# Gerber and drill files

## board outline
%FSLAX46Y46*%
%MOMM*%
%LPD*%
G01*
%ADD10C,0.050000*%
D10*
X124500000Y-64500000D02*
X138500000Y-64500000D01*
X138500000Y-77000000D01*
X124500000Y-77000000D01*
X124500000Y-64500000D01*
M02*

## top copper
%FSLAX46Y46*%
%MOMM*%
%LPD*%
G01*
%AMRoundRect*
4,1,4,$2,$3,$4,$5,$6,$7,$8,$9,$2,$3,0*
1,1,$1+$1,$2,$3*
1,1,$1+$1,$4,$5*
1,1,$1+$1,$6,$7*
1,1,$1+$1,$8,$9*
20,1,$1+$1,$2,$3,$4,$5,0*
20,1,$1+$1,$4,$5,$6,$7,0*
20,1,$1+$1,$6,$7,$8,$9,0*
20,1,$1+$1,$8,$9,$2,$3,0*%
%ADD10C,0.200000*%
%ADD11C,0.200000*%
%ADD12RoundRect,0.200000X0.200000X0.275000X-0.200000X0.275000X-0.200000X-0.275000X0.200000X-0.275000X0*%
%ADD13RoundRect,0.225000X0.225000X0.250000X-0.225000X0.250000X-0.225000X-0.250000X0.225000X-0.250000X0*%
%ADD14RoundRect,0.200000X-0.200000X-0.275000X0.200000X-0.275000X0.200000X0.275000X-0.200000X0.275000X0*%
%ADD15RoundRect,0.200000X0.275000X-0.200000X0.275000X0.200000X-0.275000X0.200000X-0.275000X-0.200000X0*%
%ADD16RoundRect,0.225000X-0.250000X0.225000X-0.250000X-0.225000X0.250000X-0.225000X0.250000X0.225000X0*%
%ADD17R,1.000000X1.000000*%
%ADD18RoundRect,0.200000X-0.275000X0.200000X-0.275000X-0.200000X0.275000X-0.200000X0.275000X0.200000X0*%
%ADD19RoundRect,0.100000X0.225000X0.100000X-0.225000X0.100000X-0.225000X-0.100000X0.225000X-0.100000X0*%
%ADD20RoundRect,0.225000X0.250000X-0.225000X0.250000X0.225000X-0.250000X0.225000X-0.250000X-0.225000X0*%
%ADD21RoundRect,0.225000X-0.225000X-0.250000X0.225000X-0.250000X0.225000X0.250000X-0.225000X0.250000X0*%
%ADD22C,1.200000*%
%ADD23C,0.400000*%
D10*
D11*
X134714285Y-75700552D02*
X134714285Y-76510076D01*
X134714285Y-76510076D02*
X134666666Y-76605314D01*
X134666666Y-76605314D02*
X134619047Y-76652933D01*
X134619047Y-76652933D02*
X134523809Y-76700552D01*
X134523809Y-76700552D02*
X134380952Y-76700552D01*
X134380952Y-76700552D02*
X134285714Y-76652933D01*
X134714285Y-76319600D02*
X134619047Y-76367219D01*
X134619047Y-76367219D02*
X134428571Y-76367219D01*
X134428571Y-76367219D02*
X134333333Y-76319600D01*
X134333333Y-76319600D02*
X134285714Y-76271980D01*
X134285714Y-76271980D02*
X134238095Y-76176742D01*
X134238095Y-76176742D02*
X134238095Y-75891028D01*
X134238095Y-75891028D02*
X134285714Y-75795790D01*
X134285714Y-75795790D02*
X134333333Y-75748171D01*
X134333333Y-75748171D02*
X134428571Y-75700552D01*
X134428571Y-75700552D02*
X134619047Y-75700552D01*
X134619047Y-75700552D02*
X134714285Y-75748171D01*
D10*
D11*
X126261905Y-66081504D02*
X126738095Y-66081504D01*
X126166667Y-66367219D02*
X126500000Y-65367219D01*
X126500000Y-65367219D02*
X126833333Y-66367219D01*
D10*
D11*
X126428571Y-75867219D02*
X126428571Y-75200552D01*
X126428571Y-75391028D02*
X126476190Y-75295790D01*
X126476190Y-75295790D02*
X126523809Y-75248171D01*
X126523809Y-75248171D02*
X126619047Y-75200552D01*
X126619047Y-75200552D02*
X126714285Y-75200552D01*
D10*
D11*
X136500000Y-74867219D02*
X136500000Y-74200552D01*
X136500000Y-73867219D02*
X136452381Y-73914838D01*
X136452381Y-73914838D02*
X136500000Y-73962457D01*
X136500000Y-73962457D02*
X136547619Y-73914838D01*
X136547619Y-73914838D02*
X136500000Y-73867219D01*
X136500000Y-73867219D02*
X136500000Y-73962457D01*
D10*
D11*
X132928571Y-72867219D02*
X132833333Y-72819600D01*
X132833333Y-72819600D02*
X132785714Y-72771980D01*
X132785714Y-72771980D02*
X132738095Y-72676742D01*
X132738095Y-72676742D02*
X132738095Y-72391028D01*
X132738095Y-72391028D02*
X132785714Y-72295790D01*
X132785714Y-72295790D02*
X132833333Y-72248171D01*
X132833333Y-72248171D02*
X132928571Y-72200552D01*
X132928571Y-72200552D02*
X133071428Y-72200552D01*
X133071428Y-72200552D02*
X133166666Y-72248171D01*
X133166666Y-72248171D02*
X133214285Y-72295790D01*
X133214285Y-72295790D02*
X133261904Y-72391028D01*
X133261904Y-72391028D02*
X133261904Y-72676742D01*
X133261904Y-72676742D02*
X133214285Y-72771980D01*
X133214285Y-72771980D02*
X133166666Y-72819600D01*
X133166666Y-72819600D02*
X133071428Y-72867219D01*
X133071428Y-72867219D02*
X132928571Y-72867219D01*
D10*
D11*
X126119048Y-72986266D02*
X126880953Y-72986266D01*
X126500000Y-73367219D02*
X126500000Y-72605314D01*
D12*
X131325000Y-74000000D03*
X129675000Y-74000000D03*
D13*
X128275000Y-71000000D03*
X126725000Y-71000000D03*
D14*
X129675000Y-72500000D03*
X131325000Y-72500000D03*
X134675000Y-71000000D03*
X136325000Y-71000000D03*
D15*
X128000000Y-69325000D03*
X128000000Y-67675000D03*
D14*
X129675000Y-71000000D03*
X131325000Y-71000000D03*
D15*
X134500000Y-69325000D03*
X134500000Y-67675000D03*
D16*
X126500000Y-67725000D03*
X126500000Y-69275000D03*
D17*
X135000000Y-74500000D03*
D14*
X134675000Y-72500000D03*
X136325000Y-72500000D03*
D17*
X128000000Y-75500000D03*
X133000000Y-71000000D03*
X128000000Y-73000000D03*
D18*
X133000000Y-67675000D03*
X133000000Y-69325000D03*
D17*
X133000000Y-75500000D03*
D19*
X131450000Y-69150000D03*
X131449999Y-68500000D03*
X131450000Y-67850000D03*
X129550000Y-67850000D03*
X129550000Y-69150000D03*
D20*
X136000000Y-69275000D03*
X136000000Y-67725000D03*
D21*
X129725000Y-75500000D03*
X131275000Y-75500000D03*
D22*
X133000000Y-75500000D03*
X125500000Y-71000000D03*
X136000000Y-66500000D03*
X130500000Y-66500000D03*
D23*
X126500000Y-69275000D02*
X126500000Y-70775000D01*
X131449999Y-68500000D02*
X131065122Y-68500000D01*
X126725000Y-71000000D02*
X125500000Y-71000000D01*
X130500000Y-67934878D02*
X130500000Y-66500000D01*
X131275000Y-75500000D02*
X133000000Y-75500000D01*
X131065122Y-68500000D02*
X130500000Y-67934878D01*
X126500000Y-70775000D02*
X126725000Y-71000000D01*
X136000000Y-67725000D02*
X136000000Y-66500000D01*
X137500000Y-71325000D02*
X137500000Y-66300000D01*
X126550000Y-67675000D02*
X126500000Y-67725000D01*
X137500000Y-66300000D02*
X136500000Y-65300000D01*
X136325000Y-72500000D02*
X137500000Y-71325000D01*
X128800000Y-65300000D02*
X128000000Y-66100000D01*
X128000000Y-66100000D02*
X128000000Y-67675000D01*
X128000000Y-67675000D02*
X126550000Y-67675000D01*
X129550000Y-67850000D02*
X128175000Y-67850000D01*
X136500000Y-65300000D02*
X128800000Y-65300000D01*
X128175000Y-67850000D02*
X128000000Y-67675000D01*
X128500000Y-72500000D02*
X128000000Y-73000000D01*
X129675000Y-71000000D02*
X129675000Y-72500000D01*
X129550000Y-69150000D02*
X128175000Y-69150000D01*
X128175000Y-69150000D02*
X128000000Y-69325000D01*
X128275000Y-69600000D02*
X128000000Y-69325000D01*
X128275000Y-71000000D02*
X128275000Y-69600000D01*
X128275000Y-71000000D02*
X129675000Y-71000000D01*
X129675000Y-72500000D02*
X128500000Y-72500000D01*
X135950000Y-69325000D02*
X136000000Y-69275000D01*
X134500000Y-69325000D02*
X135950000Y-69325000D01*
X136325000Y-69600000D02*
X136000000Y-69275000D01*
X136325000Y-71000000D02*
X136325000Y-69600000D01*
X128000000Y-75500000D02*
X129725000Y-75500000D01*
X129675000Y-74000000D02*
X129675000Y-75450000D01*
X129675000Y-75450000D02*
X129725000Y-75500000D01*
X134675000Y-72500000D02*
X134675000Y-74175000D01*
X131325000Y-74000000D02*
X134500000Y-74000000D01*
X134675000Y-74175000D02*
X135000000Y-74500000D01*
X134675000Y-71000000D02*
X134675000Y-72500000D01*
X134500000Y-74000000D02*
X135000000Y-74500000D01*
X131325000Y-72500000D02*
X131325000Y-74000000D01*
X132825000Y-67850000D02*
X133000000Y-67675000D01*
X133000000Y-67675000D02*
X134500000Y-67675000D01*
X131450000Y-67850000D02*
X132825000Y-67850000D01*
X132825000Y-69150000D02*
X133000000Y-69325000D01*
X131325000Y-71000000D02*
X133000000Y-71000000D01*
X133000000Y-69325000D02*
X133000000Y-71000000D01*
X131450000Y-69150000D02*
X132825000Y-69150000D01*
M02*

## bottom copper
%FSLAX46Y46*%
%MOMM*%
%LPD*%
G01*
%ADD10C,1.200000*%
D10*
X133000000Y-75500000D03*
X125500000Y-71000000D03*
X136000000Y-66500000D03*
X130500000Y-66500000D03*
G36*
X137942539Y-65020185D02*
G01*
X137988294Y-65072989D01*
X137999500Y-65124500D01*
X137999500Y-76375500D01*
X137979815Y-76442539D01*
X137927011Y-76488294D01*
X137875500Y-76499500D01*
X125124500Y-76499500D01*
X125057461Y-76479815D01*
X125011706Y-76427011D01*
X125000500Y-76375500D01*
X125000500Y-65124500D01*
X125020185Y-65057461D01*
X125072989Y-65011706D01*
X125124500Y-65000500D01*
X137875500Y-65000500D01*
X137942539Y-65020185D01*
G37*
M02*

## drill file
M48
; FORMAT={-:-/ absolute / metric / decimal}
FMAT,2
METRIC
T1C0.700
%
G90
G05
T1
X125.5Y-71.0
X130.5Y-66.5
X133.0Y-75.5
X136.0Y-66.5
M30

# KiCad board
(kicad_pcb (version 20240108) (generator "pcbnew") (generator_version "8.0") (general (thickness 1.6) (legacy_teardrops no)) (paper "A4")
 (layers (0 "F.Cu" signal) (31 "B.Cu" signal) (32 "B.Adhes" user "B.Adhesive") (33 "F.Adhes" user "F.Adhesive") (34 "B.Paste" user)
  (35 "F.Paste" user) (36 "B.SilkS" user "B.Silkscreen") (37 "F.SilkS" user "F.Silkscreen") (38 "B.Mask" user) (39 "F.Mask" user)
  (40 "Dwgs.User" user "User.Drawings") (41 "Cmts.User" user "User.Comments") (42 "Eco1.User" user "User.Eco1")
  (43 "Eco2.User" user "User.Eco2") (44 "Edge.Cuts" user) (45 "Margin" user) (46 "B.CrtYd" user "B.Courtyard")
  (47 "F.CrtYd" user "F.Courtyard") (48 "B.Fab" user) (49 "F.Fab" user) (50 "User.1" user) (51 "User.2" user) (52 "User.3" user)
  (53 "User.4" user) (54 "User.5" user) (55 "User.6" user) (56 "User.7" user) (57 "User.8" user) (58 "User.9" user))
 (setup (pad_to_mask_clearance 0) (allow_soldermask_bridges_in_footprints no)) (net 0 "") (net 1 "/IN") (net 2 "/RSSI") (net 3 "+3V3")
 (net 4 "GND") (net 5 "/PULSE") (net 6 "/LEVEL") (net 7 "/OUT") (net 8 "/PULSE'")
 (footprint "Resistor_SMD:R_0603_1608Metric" (layer "F.Cu") (at 130.5 74 180)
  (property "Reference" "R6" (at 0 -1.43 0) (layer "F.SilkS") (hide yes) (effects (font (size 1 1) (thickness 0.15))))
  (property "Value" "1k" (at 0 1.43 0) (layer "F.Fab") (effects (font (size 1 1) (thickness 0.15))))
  (pad "1" smd roundrect (at -0.825 0 180) (size 0.8 0.95) (layers "F.Cu" "F.Paste" "F.Mask") (roundrect_rratio 0.25) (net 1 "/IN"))
  (pad "2" smd roundrect (at 0.825 0 180) (size 0.8 0.95) (layers "F.Cu" "F.Paste" "F.Mask") (roundrect_rratio 0.25) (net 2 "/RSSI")))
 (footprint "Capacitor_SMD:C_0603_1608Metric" (layer "F.Cu") (at 127.5 71 180)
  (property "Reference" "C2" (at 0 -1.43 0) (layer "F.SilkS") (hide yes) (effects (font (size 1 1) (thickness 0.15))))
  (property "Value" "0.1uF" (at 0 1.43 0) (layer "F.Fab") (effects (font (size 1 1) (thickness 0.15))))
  (pad "1" smd roundrect (at -0.775 0 180) (size 0.9 0.95) (layers "F.Cu" "F.Paste" "F.Mask") (roundrect_rratio 0.25) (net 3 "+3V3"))
  (pad "2" smd roundrect (at 0.775 0 180) (size 0.9 0.95) (layers "F.Cu" "F.Paste" "F.Mask") (roundrect_rratio 0.25) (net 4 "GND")))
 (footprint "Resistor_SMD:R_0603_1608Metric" (layer "F.Cu") (at 130.5 72.5)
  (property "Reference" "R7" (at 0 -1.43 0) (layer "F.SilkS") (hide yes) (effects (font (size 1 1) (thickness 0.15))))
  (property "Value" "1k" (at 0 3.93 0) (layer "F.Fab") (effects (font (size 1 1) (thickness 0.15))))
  (pad "1" smd roundrect (at -0.825 0) (size 0.8 0.95) (layers "F.Cu" "F.Paste" "F.Mask") (roundrect_rratio 0.25) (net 3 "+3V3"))
  (pad "2" smd roundrect (at 0.825 0) (size 0.8 0.95) (layers "F.Cu" "F.Paste" "F.Mask") (roundrect_rratio 0.25) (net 1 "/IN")))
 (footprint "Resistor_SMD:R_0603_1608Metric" (layer "F.Cu") (at 135.5 71)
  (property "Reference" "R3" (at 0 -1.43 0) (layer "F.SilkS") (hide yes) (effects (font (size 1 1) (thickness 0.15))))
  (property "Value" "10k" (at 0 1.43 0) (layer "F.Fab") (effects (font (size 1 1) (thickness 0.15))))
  (pad "1" smd roundrect (at -0.825 0) (size 0.8 0.95) (layers "F.Cu" "F.Paste" "F.Mask") (roundrect_rratio 0.25) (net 1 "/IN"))
  (pad "2" smd roundrect (at 0.825 0) (size 0.8 0.95) (layers "F.Cu" "F.Paste" "F.Mask") (roundrect_rratio 0.25) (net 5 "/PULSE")))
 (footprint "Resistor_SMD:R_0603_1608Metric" (layer "F.Cu") (at 128 68.5 90)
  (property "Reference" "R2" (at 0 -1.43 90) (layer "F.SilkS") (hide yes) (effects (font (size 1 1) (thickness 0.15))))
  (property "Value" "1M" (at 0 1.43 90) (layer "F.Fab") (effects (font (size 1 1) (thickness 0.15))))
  (pad "1" smd roundrect (at -0.825 0 90) (size 0.8 0.95) (layers "F.Cu" "F.Paste" "F.Mask") (roundrect_rratio 0.25) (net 3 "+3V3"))
  (pad "2" smd roundrect (at 0.825 0 90) (size 0.8 0.95) (layers "F.Cu" "F.Paste" "F.Mask") (roundrect_rratio 0.25) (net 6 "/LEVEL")))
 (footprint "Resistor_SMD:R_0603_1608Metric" (layer "F.Cu") (at 130.5 71)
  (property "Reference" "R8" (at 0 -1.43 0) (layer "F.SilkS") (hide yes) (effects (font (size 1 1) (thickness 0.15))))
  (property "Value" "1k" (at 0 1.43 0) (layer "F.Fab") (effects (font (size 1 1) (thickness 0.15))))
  (pad "1" smd roundrect (at -0.825 0) (size 0.8 0.95) (layers "F.Cu" "F.Paste" "F.Mask") (roundrect_rratio 0.25) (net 3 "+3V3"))
  (pad "2" smd roundrect (at 0.825 0) (size 0.8 0.95) (layers "F.Cu" "F.Paste" "F.Mask") (roundrect_rratio 0.25) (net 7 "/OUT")))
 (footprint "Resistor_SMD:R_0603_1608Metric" (layer "F.Cu") (at 134.5 68.5 90)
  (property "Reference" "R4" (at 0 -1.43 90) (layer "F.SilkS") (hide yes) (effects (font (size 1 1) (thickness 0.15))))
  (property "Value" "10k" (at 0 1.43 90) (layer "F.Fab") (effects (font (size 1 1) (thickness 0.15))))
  (pad "1" smd roundrect (at -0.825 0 90) (size 0.8 0.95) (layers "F.Cu" "F.Paste" "F.Mask") (roundrect_rratio 0.25) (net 5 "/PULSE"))
  (pad "2" smd roundrect (at 0.825 0 90) (size 0.8 0.95) (layers "F.Cu" "F.Paste" "F.Mask") (roundrect_rratio 0.25) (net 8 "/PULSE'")))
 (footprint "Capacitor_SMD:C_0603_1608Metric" (layer "F.Cu") (at 126.5 68.5 -90)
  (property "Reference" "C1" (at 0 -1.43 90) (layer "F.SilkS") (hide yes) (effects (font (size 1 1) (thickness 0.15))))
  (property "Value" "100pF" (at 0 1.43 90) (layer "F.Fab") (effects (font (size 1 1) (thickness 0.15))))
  (pad "1" smd roundrect (at -0.775 0 270) (size 0.9 0.95) (layers "F.Cu" "F.Paste" "F.Mask") (roundrect_rratio 0.25) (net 6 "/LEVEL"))
  (pad "2" smd roundrect (at 0.775 0 270) (size 0.9 0.95) (layers "F.Cu" "F.Paste" "F.Mask") (roundrect_rratio 0.25) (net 4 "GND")))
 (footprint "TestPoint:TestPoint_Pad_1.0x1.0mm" (layer "F.Cu") (at 135 74.5)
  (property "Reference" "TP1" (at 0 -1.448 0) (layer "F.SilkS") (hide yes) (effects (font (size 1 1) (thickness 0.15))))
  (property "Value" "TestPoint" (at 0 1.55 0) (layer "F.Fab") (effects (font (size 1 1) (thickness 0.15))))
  (pad "1" smd rect (at 0 0) (size 1 1) (layers "F.Cu" "F.Mask") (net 1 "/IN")))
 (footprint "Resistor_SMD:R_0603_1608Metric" (layer "F.Cu") (at 135.5 72.5)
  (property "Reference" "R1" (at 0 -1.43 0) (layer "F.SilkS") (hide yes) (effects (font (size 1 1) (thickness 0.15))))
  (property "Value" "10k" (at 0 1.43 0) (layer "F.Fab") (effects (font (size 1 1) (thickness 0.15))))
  (pad "1" smd roundrect (at -0.825 0) (size 0.8 0.95) (layers "F.Cu" "F.Paste" "F.Mask") (roundrect_rratio 0.25) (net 1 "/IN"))
  (pad "2" smd roundrect (at 0.825 0) (size 0.8 0.95) (layers "F.Cu" "F.Paste" "F.Mask") (roundrect_rratio 0.25) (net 6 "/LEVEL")))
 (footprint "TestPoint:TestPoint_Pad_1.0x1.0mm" (layer "F.Cu") (at 128 75.5)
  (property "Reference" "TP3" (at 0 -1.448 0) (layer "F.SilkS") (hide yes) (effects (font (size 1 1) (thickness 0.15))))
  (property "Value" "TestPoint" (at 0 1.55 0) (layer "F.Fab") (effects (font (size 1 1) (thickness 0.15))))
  (pad "1" smd rect (at 0 0) (size 1 1) (layers "F.Cu" "F.Mask") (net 2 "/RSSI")))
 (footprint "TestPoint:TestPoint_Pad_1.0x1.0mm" (layer "F.Cu") (at 133 71)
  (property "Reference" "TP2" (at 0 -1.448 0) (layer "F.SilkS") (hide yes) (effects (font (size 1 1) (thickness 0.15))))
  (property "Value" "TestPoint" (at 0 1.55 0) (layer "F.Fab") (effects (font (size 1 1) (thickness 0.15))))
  (pad "1" smd rect (at 0 0) (size 1 1) (layers "F.Cu" "F.Mask") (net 7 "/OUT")))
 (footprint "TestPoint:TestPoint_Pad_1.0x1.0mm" (layer "F.Cu") (at 128 73)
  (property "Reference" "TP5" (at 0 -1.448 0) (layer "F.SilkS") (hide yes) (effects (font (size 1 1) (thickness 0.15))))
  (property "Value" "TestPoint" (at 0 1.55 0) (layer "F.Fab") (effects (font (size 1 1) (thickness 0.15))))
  (pad "1" smd rect (at 0 0) (size 1 1) (layers "F.Cu" "F.Mask") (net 3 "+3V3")))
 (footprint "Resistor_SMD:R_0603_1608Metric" (layer "F.Cu") (at 133 68.5 -90)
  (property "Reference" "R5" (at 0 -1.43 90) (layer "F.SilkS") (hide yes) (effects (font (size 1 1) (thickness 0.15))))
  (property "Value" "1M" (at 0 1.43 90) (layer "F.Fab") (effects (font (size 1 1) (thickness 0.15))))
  (pad "1" smd roundrect (at -0.825 0 270) (size 0.8 0.95) (layers "F.Cu" "F.Paste" "F.Mask") (roundrect_rratio 0.25) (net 8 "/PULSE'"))
  (pad "2" smd roundrect (at 0.825 0 270) (size 0.8 0.95) (layers "F.Cu" "F.Paste" "F.Mask") (roundrect_rratio 0.25) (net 7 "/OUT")))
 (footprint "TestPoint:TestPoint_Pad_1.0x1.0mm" (layer "F.Cu") (at 133 75.5)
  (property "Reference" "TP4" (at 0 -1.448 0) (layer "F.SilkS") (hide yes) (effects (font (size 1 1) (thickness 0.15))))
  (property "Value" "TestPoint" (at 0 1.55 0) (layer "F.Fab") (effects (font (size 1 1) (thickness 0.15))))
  (pad "1" smd rect (at 0 0) (size 1 1) (layers "F.Cu" "F.Mask") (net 4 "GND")))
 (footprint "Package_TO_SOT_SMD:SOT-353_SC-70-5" (layer "F.Cu") (at 130.5 68.5 180)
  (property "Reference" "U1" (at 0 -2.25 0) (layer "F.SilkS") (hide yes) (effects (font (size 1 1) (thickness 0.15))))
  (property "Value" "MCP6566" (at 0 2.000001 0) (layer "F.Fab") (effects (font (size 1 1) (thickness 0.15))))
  (pad "1" smd roundrect (at -0.95 -0.65 180) (size 0.65 0.4) (layers "F.Cu" "F.Paste" "F.Mask") (roundrect_rratio 0.25) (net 7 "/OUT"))
  (pad "2" smd roundrect (at -0.949999 0 180) (size 0.65 0.4) (layers "F.Cu" "F.Paste" "F.Mask") (roundrect_rratio 0.25) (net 4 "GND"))
  (pad "3" smd roundrect (at -0.95 0.65 180) (size 0.65 0.4) (layers "F.Cu" "F.Paste" "F.Mask") (roundrect_rratio 0.25) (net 8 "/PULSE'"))
  (pad "4" smd roundrect (at 0.95 0.65 180) (size 0.65 0.4) (layers "F.Cu" "F.Paste" "F.Mask") (roundrect_rratio 0.25) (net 6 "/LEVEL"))
  (pad "5" smd roundrect (at 0.95 -0.65 180) (size 0.65 0.4) (layers "F.Cu" "F.Paste" "F.Mask") (roundrect_rratio 0.25) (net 3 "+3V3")))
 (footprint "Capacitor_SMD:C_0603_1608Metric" (layer "F.Cu") (at 136 68.5 90)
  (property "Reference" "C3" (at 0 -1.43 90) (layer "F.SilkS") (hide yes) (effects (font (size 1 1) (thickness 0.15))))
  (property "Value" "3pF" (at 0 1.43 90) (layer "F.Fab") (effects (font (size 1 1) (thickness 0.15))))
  (pad "1" smd roundrect (at -0.775 0 90) (size 0.9 0.95) (layers "F.Cu" "F.Paste" "F.Mask") (roundrect_rratio 0.25) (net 5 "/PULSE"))
  (pad "2" smd roundrect (at 0.775 0 90) (size 0.9 0.95) (layers "F.Cu" "F.Paste" "F.Mask") (roundrect_rratio 0.25) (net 4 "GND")))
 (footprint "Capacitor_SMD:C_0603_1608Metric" (layer "F.Cu") (at 130.5 75.5)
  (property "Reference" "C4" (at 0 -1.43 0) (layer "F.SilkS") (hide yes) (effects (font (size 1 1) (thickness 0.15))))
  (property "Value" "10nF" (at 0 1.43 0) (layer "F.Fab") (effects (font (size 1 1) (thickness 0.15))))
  (pad "1" smd roundrect (at -0.775 0) (size 0.9 0.95) (layers "F.Cu" "F.Paste" "F.Mask") (roundrect_rratio 0.25) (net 2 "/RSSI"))
  (pad "2" smd roundrect (at 0.775 0) (size 0.9 0.95) (layers "F.Cu" "F.Paste" "F.Mask") (roundrect_rratio 0.25) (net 4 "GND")))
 (gr_rect (start 124.5 64.5) (end 138.5 77) (stroke (width 0.05) (type default)) (fill none) (layer "Edge.Cuts"))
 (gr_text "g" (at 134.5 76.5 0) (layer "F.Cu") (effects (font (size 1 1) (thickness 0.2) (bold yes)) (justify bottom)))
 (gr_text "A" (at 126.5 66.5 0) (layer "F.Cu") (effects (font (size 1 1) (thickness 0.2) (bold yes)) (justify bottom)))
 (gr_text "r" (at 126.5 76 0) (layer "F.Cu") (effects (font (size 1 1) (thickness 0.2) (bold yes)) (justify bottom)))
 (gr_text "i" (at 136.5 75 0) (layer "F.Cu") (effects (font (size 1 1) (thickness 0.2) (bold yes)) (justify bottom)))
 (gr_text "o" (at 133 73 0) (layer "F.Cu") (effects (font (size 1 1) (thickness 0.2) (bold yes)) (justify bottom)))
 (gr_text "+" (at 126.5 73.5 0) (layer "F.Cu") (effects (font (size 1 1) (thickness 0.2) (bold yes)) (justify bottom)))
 (segment (start 126.5 69.275) (end 126.5 70.775) (width 0.4) (layer "F.Cu") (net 4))
 (segment (start 131.449999 68.5) (end 131.065122 68.5) (width 0.4) (layer "F.Cu") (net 4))
 (segment (start 126.725 71) (end 125.5 71) (width 0.4) (layer "F.Cu") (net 4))
 (segment (start 130.5 67.934878) (end 130.5 66.5) (width 0.4) (layer "F.Cu") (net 4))
 (segment (start 131.275 75.5) (end 133 75.5) (width 0.4) (layer "F.Cu") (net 4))
 (segment (start 131.065122 68.5) (end 130.5 67.934878) (width 0.4) (layer "F.Cu") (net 4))
 (segment (start 126.5 70.775) (end 126.725 71) (width 0.4) (layer "F.Cu") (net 4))
 (segment (start 136 67.725) (end 136 66.5) (width 0.4) (layer "F.Cu") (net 4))
 (via (at 133 75.5) (size 1.2) (drill 0.7) (layers "F.Cu" "B.Cu") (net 4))
 (via (at 125.5 71) (size 1.2) (drill 0.7) (layers "F.Cu" "B.Cu") (free yes) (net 4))
 (via (at 136 66.5) (size 1.2) (drill 0.7) (layers "F.Cu" "B.Cu") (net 4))
 (via (at 130.5 66.5) (size 1.2) (drill 0.7) (layers "F.Cu" "B.Cu") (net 4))
 (segment (start 137.5 71.325) (end 137.5 66.3) (width 0.4) (layer "F.Cu") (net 6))
 (segment (start 126.55 67.675) (end 126.5 67.725) (width 0.4) (layer "F.Cu") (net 6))
 (segment (start 137.5 66.3) (end 136.5 65.3) (width 0.4) (layer "F.Cu") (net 6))
 (segment (start 136.325 72.5) (end 137.5 71.325) (width 0.4) (layer "F.Cu") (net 6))
 (segment (start 128.8 65.3) (end 128 66.1) (width 0.4) (layer "F.Cu") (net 6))
 (segment (start 128 66.1) (end 128 67.675) (width 0.4) (layer "F.Cu") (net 6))
 (segment (start 128 67.675) (end 126.55 67.675) (width 0.4) (layer "F.Cu") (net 6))
 (segment (start 129.55 67.85) (end 128.175 67.85) (width 0.4) (layer "F.Cu") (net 6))
 (segment (start 136.5 65.3) (end 128.8 65.3) (width 0.4) (layer "F.Cu") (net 6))
 (segment (start 128.175 67.85) (end 128 67.675) (width 0.4) (layer "F.Cu") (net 6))
 (segment (start 128.5 72.5) (end 128 73) (width 0.4) (layer "F.Cu") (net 3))
 (segment (start 129.675 71) (end 129.675 72.5) (width 0.4) (layer "F.Cu") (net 3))
 (segment (start 129.55 69.15) (end 128.175 69.15) (width 0.4) (layer "F.Cu") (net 3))
 (segment (start 128.175 69.15) (end 128 69.325) (width 0.4) (layer "F.Cu") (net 3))
 (segment (start 128.275 69.6) (end 128 69.325) (width 0.4) (layer "F.Cu") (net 3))
 (segment (start 128.275 71) (end 128.275 69.6) (width 0.4) (layer "F.Cu") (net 3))
 (segment (start 128.275 71) (end 129.675 71) (width 0.4) (layer "F.Cu") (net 3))
 (segment (start 129.675 72.5) (end 128.5 72.5) (width 0.4) (layer "F.Cu") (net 3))
 (segment (start 135.95 69.325) (end 136 69.275) (width 0.4) (layer "F.Cu") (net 5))
 (segment (start 134.5 69.325) (end 135.95 69.325) (width 0.4) (layer "F.Cu") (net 5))
 (segment (start 136.325 69.6) (end 136 69.275) (width 0.4) (layer "F.Cu") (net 5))
 (segment (start 136.325 71) (end 136.325 69.6) (width 0.4) (layer "F.Cu") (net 5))
 (segment (start 128 75.5) (end 129.725 75.5) (width 0.4) (layer "F.Cu") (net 2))
 (segment (start 129.675 74) (end 129.675 75.45) (width 0.4) (layer "F.Cu") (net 2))
 (segment (start 129.675 75.45) (end 129.725 75.5) (width 0.4) (layer "F.Cu") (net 2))
 (segment (start 134.675 72.5) (end 134.675 74.175) (width 0.4) (layer "F.Cu") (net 1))
 (segment (start 131.325 74) (end 134.5 74) (width 0.4) (layer "F.Cu") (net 1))
 (segment (start 134.675 74.175) (end 135 74.5) (width 0.4) (layer "F.Cu") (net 1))
 (segment (start 134.675 71) (end 134.675 72.5) (width 0.4) (layer "F.Cu") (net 1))
 (segment (start 134.5 74) (end 135 74.5) (width 0.4) (layer "F.Cu") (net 1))
 (segment (start 131.325 72.5) (end 131.325 74) (width 0.4) (layer "F.Cu") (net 1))
 (segment (start 132.825 67.85) (end 133 67.675) (width 0.4) (layer "F.Cu") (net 8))
 (segment (start 133 67.675) (end 134.5 67.675) (width 0.4) (layer "F.Cu") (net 8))
 (segment (start 131.45 67.85) (end 132.825 67.85) (width 0.4) (layer "F.Cu") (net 8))
 (segment (start 132.825 69.15) (end 133 69.325) (width 0.4) (layer "F.Cu") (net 7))
 (segment (start 131.325 71) (end 133 71) (width 0.4) (layer "F.Cu") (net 7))
 (segment (start 133 69.325) (end 133 71) (width 0.4) (layer "F.Cu") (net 7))
 (segment (start 131.45 69.15) (end 132.825 69.15) (width 0.4) (layer "F.Cu") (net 7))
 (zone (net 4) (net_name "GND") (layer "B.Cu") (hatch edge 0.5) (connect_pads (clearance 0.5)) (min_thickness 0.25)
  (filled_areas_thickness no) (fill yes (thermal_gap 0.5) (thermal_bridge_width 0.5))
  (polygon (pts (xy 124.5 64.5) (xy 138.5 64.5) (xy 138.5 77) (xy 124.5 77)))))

